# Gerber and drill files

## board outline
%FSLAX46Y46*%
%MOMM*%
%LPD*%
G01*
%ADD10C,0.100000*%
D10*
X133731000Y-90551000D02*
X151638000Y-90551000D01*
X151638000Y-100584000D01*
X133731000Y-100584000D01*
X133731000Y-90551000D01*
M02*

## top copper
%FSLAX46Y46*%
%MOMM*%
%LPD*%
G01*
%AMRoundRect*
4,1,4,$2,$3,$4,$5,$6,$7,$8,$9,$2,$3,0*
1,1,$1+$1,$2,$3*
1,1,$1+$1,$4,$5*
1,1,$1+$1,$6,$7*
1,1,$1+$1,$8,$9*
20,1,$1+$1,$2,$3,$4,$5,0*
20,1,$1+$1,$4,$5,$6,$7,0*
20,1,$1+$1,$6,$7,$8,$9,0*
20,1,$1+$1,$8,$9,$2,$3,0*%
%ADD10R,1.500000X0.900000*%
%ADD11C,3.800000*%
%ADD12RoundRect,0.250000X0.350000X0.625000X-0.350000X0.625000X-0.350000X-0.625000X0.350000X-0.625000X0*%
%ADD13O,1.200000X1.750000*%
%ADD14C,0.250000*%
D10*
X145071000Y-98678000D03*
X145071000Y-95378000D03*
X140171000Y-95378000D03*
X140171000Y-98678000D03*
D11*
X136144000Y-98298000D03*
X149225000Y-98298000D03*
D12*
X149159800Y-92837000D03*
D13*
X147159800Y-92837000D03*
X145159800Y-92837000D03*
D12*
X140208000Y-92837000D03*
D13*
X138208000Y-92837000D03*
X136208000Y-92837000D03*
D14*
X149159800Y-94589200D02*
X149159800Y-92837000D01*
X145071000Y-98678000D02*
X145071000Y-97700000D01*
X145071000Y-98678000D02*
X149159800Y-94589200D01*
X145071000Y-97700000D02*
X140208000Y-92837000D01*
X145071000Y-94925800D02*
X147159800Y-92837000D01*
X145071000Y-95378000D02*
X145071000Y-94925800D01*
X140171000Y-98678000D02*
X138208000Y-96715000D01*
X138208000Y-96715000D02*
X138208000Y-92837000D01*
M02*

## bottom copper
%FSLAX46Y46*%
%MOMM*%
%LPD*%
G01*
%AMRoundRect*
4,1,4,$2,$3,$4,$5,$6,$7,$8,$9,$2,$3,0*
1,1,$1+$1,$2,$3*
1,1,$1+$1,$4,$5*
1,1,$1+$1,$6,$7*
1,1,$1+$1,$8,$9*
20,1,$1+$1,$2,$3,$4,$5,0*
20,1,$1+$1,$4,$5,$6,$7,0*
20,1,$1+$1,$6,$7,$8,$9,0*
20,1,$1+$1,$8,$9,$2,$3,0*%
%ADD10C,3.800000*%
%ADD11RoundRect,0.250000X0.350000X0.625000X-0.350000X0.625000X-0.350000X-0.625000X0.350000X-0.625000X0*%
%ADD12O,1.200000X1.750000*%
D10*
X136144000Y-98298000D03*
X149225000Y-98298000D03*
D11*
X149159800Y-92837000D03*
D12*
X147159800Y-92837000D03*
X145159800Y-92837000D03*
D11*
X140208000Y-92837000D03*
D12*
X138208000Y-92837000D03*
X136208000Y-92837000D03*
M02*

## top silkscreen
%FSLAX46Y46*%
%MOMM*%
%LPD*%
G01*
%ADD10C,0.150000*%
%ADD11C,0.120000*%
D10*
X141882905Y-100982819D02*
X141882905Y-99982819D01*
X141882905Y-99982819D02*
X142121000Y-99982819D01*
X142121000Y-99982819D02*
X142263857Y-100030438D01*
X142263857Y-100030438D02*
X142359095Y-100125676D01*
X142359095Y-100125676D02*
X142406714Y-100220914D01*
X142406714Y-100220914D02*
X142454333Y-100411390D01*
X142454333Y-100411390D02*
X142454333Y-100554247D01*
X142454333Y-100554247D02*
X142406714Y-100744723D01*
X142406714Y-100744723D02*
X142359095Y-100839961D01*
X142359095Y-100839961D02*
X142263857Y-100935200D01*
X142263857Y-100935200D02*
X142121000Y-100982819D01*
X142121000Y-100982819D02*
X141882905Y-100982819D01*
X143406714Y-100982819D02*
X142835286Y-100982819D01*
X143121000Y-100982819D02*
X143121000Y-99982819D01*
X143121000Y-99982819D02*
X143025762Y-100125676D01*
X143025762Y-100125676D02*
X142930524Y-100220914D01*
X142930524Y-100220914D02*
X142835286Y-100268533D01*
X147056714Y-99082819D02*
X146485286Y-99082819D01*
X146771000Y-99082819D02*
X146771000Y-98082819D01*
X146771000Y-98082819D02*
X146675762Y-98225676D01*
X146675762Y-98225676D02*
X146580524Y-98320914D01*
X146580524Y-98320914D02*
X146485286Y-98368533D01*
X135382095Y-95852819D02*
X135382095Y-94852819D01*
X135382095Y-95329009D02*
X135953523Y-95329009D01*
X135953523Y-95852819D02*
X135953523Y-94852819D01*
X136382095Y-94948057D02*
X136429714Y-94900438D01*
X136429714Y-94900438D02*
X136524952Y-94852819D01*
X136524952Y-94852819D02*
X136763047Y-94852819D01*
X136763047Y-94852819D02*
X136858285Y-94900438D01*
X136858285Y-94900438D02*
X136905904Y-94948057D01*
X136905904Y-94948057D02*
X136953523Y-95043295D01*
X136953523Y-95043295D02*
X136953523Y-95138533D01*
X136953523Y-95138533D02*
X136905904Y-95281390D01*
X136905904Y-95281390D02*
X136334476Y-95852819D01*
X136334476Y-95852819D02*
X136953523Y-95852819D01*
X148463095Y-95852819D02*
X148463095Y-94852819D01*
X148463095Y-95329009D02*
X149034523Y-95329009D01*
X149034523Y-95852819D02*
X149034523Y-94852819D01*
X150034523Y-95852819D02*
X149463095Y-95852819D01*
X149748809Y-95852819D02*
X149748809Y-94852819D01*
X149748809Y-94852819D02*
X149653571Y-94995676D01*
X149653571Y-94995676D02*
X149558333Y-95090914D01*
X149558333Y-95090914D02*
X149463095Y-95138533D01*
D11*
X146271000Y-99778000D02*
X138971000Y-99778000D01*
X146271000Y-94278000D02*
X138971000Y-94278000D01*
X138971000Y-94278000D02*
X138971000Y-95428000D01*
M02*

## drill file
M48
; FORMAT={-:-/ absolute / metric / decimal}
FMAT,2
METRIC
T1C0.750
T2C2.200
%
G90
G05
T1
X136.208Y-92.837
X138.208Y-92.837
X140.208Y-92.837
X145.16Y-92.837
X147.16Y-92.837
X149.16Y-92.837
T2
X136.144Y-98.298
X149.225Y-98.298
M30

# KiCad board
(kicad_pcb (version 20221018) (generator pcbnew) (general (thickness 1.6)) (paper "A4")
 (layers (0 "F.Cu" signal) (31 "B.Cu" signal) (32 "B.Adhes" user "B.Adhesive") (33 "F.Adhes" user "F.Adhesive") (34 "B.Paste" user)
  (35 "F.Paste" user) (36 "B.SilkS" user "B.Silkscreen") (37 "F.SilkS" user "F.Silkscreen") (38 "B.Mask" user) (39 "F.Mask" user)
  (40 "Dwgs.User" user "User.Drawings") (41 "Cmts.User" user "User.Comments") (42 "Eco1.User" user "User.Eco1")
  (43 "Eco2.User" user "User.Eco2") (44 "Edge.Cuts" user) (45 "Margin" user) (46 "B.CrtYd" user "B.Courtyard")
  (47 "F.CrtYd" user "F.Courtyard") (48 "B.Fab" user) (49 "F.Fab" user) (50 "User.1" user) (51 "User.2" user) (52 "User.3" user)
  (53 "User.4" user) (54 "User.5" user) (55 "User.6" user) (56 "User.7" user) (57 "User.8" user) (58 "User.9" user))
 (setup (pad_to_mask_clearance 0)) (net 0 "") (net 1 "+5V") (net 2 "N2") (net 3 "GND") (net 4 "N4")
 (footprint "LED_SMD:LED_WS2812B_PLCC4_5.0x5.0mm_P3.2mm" (layer "F.Cu") (at 142.621 97.028 180)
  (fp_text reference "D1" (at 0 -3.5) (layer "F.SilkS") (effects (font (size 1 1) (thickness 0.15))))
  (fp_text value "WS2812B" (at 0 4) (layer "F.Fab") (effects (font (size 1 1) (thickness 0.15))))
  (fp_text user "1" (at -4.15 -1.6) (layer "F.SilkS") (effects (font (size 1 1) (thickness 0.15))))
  (fp_line (start -3.65 -2.75) (end 3.65 -2.75) (stroke (width 0.12) (type solid)) (layer "F.SilkS"))
  (fp_line (start -3.65 2.75) (end 3.65 2.75) (stroke (width 0.12) (type solid)) (layer "F.SilkS"))
  (fp_line (start 3.65 2.75) (end 3.65 1.6) (stroke (width 0.12) (type solid)) (layer "F.SilkS"))
  (pad "1" smd rect (at -2.45 -1.65 180) (size 1.5 0.9) (layers "F.Cu" "F.Paste" "F.Mask") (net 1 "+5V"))
  (pad "2" smd rect (at -2.45 1.65 180) (size 1.5 0.9) (layers "F.Cu" "F.Paste" "F.Mask") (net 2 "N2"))
  (pad "3" smd rect (at 2.45 1.65 180) (size 1.5 0.9) (layers "F.Cu" "F.Paste" "F.Mask") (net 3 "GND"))
  (pad "4" smd rect (at 2.45 -1.65 180) (size 1.5 0.9) (layers "F.Cu" "F.Paste" "F.Mask") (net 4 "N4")))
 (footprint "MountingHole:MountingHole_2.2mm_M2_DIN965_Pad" (layer "F.Cu") (at 136.144 98.298)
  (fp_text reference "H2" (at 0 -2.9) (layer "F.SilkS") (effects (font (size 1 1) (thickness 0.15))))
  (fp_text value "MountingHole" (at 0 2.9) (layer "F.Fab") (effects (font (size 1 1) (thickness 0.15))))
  (pad "1" thru_hole circle (at 0 0) (size 3.8 3.8) (drill 2.2) (layers "*.Cu" "*.Mask")))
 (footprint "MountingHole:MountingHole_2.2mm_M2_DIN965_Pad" (layer "F.Cu") (at 149.225 98.298)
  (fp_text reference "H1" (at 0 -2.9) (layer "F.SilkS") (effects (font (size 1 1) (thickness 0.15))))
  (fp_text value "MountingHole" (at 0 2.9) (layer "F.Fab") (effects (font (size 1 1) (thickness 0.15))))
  (pad "1" thru_hole circle (at 0 0) (size 3.8 3.8) (drill 2.2) (layers "*.Cu" "*.Mask")))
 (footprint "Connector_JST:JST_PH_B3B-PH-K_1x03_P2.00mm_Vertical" (layer "B.Cu") (at 149.1598 92.837 180)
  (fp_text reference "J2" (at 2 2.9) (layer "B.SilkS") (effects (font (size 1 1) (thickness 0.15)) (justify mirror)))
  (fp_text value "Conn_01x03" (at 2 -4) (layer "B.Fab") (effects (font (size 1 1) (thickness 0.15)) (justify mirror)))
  (pad "1" thru_hole roundrect (at 0 0 180) (size 1.2 1.75) (drill 0.75) (layers "*.Cu" "*.Mask") (roundrect_rratio 0.208333) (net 1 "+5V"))
  (pad "2" thru_hole oval (at 2 0 180) (size 1.2 1.75) (drill 0.75) (layers "*.Cu" "*.Mask") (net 2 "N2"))
  (pad "3" thru_hole oval (at 4 0 180) (size 1.2 1.75) (drill 0.75) (layers "*.Cu" "*.Mask") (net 3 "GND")))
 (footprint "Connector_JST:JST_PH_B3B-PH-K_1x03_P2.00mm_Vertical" (layer "B.Cu") (at 140.208 92.837 180)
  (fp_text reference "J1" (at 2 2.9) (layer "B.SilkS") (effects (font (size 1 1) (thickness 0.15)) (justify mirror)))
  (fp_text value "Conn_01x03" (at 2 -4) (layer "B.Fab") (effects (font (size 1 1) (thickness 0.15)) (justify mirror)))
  (pad "1" thru_hole roundrect (at 0 0 180) (size 1.2 1.75) (drill 0.75) (layers "*.Cu" "*.Mask") (roundrect_rratio 0.208333) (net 1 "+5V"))
  (pad "2" thru_hole oval (at 2 0 180) (size 1.2 1.75) (drill 0.75) (layers "*.Cu" "*.Mask") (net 4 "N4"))
  (pad "3" thru_hole oval (at 4 0 180) (size 1.2 1.75) (drill 0.75) (layers "*.Cu" "*.Mask") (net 3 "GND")))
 (gr_rect (start 133.731 90.551) (end 151.638 100.584) (stroke (width 0.1) (type default)) (fill none) (layer "Edge.Cuts"))
 (segment (start 149.1598 94.5892) (end 149.1598 92.837) (width 0.25) (layer "F.Cu") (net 1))
 (segment (start 145.071 98.678) (end 145.071 97.7) (width 0.25) (layer "F.Cu") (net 1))
 (segment (start 145.071 98.678) (end 149.1598 94.5892) (width 0.25) (layer "F.Cu") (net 1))
 (segment (start 145.071 97.7) (end 140.208 92.837) (width 0.25) (layer "F.Cu") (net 1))
 (segment (start 145.071 94.9258) (end 147.1598 92.837) (width 0.25) (layer "F.Cu") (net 2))
 (segment (start 145.071 95.378) (end 145.071 94.9258) (width 0.25) (layer "F.Cu") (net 2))
 (segment (start 140.171 98.678) (end 138.208 96.715) (width 0.25) (layer "F.Cu") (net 4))
 (segment (start 138.208 96.715) (end 138.208 92.837) (width 0.25) (layer "F.Cu") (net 4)))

